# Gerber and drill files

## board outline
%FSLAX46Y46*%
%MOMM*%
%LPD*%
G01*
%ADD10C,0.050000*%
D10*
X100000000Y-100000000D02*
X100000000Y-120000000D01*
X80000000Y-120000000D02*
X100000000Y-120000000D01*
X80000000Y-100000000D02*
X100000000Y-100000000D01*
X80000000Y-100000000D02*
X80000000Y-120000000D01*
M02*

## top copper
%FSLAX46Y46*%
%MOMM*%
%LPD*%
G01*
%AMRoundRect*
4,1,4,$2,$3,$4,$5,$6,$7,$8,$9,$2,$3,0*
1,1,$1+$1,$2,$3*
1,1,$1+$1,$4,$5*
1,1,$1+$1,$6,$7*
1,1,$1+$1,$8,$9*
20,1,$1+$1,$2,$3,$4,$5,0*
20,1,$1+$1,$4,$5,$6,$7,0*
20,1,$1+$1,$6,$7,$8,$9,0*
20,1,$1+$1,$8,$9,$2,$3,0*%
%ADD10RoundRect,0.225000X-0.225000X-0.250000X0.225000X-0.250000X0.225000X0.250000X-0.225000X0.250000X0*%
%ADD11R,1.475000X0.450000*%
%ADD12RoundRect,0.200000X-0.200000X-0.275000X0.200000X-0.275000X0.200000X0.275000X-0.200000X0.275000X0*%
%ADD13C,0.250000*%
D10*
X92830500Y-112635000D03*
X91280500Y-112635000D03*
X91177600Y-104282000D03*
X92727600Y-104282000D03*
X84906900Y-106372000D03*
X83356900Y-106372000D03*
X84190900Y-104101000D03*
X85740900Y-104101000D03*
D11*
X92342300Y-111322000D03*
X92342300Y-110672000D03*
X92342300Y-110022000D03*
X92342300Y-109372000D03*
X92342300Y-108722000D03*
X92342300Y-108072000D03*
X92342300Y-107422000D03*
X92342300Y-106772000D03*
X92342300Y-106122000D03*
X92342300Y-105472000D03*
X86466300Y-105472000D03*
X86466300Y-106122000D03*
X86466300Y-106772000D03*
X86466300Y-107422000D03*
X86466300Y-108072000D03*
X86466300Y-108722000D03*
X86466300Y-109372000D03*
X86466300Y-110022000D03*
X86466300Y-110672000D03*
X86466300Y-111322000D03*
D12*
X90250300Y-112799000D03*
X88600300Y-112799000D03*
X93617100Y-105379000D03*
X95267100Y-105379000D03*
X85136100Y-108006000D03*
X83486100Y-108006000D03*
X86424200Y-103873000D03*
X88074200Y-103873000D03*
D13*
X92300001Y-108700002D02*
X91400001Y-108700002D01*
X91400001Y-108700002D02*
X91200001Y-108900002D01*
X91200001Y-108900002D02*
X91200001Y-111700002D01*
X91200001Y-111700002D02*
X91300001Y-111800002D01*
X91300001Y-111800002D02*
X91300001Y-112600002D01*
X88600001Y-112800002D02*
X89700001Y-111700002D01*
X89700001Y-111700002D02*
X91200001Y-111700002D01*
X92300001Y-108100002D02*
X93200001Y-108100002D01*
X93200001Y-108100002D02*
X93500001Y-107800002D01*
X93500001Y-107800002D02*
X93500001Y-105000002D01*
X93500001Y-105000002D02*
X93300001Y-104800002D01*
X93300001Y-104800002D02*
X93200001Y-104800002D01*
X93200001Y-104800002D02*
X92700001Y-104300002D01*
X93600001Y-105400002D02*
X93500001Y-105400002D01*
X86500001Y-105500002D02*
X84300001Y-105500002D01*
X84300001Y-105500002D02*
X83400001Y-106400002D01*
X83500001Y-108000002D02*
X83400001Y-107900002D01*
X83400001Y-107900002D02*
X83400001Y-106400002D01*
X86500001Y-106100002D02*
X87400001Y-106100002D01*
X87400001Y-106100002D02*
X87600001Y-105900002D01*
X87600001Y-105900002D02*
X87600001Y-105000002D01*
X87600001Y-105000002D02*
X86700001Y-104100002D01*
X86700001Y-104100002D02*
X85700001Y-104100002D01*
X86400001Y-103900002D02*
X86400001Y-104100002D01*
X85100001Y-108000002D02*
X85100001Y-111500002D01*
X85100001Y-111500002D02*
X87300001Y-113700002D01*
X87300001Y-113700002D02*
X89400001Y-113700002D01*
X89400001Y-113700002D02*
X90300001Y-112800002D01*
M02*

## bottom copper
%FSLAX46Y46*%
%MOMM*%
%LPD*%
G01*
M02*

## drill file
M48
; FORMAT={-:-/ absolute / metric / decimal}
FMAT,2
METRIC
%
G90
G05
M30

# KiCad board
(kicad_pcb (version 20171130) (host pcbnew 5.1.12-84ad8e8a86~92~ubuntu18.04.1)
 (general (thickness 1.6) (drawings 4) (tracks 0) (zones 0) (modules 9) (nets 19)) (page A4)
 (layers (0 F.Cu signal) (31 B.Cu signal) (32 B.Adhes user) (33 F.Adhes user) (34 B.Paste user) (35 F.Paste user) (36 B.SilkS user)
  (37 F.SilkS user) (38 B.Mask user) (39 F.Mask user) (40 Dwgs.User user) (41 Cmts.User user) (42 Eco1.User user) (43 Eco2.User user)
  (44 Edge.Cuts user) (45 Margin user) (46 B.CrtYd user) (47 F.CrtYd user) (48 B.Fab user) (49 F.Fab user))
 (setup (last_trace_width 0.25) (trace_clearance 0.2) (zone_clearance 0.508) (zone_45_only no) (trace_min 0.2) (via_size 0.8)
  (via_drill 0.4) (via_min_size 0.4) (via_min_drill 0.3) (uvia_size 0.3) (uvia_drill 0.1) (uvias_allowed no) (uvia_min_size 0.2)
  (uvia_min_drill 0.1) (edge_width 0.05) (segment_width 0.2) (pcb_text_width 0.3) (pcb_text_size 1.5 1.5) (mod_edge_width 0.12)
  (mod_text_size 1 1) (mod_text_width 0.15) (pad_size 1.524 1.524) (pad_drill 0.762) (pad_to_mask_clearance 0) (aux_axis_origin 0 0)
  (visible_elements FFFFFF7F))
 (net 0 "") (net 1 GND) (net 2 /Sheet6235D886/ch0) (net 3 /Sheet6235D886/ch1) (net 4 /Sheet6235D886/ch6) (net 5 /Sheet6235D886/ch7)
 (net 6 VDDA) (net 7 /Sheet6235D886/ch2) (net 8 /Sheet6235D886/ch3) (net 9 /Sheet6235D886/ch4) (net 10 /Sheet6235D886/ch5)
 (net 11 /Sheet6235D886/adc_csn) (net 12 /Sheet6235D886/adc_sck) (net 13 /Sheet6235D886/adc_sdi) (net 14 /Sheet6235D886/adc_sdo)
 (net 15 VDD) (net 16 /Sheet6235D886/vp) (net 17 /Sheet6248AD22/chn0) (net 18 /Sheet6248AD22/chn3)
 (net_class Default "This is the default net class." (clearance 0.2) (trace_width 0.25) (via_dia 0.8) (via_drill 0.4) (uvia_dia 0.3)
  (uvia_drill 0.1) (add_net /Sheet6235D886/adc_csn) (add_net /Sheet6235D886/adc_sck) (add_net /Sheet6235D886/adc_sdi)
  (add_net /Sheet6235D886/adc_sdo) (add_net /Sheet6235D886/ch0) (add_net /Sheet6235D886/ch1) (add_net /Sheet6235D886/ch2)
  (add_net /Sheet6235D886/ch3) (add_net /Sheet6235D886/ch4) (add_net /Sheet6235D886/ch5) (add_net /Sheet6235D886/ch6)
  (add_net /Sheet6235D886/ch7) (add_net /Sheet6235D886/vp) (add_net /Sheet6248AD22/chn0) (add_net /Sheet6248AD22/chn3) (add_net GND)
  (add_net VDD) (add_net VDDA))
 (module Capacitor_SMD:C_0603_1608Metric (layer F.Cu) (at 92.055500 112.635000)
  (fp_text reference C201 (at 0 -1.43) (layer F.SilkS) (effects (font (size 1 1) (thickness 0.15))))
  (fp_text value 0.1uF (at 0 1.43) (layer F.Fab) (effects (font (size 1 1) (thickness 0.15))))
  (pad 2 smd roundrect (at 0.775 0) (size 0.9 0.95) (layers F.Cu F.Mask F.Paste) (roundrect_rratio 0.25) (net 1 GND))
  (pad 1 smd roundrect (at -0.775 0) (size 0.9 0.95) (layers F.Cu F.Mask F.Paste) (roundrect_rratio 0.25) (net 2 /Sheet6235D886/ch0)))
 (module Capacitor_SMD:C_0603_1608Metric (layer F.Cu) (at 91.952600 104.282000)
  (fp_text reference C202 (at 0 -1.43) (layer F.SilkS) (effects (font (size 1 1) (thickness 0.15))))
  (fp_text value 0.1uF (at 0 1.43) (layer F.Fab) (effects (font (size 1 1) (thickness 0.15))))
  (pad 1 smd roundrect (at -0.775 0) (size 0.9 0.95) (layers F.Cu F.Mask F.Paste) (roundrect_rratio 0.25) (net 1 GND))
  (pad 2 smd roundrect (at 0.775 0) (size 0.9 0.95) (layers F.Cu F.Mask F.Paste) (roundrect_rratio 0.25) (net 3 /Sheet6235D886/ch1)))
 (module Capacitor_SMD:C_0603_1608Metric (layer F.Cu) (at 84.131900 106.372000)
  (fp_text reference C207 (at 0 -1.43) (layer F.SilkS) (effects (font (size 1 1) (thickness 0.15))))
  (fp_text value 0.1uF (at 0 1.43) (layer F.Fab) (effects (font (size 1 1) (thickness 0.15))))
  (pad 2 smd roundrect (at 0.775 0) (size 0.9 0.95) (layers F.Cu F.Mask F.Paste) (roundrect_rratio 0.25) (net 1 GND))
  (pad 1 smd roundrect (at -0.775 0) (size 0.9 0.95) (layers F.Cu F.Mask F.Paste) (roundrect_rratio 0.25) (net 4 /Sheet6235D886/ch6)))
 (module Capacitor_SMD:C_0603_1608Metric (layer F.Cu) (at 84.965900 104.101000)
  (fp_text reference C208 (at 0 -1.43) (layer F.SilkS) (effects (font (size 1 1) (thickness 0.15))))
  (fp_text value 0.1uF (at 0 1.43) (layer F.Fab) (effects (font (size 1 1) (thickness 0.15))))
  (pad 1 smd roundrect (at -0.775 0) (size 0.9 0.95) (layers F.Cu F.Mask F.Paste) (roundrect_rratio 0.25) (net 1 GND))
  (pad 2 smd roundrect (at 0.775 0) (size 0.9 0.95) (layers F.Cu F.Mask F.Paste) (roundrect_rratio 0.25) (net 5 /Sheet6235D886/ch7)))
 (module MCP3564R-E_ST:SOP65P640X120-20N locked (layer F.Cu) (at 89.404300 108.397000 180.000000)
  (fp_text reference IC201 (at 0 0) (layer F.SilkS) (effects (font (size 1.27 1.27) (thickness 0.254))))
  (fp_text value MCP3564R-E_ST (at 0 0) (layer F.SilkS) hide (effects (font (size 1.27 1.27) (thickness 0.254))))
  (pad 1 smd rect (at -2.938 -2.925 270.000000) (size 0.45 1.475) (layers F.Cu F.Mask F.Paste) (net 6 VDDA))
  (pad 2 smd rect (at -2.938 -2.275 270.000000) (size 0.45 1.475) (layers F.Cu F.Mask F.Paste) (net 1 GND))
  (pad 3 smd rect (at -2.938 -1.625 270.000000) (size 0.45 1.475) (layers F.Cu F.Mask F.Paste) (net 1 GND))
  (pad 4 smd rect (at -2.938 -0.975 270.000000) (size 0.45 1.475) (layers F.Cu F.Mask F.Paste))
  (pad 5 smd rect (at -2.938 -0.325 270.000000) (size 0.45 1.475) (layers F.Cu F.Mask F.Paste) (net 2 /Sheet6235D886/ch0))
  (pad 6 smd rect (at -2.938 0.325 270.000000) (size 0.45 1.475) (layers F.Cu F.Mask F.Paste) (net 3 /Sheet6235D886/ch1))
  (pad 7 smd rect (at -2.938 0.975 270.000000) (size 0.45 1.475) (layers F.Cu F.Mask F.Paste) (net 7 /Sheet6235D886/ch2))
  (pad 8 smd rect (at -2.938 1.625 270.000000) (size 0.45 1.475) (layers F.Cu F.Mask F.Paste) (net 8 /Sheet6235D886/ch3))
  (pad 9 smd rect (at -2.938 2.275 270.000000) (size 0.45 1.475) (layers F.Cu F.Mask F.Paste) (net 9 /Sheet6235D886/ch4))
  (pad 10 smd rect (at -2.938 2.925 270.000000) (size 0.45 1.475) (layers F.Cu F.Mask F.Paste) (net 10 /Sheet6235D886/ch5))
  (pad 11 smd rect (at 2.938 2.925 270.000000) (size 0.45 1.475) (layers F.Cu F.Mask F.Paste) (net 4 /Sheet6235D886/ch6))
  (pad 12 smd rect (at 2.938 2.275 270.000000) (size 0.45 1.475) (layers F.Cu F.Mask F.Paste) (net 5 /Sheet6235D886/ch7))
  (pad 13 smd rect (at 2.938 1.625 270.000000) (size 0.45 1.475) (layers F.Cu F.Mask F.Paste) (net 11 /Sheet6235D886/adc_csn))
  (pad 14 smd rect (at 2.938 0.975 270.000000) (size 0.45 1.475) (layers F.Cu F.Mask F.Paste) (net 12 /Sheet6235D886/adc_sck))
  (pad 15 smd rect (at 2.938 0.325 270.000000) (size 0.45 1.475) (layers F.Cu F.Mask F.Paste) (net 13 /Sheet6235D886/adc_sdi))
  (pad 16 smd rect (at 2.938 -0.325 270.000000) (size 0.45 1.475) (layers F.Cu F.Mask F.Paste) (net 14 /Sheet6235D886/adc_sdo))
  (pad 17 smd rect (at 2.938 -0.975 270.000000) (size 0.45 1.475) (layers F.Cu F.Mask F.Paste))
  (pad 18 smd rect (at 2.938 -1.625 270.000000) (size 0.45 1.475) (layers F.Cu F.Mask F.Paste))
  (pad 19 smd rect (at 2.938 -2.275 270.000000) (size 0.45 1.475) (layers F.Cu F.Mask F.Paste) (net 1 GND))
  (pad 20 smd rect (at 2.938 -2.925 270.000000) (size 0.45 1.475) (layers F.Cu F.Mask F.Paste) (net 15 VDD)))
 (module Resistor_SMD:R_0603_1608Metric (layer F.Cu) (at 89.425300 112.799000)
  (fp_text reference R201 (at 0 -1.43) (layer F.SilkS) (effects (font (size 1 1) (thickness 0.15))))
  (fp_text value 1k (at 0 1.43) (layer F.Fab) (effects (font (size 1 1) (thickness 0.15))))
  (pad 2 smd roundrect (at 0.825 0) (size 0.8 0.95) (layers F.Cu F.Mask F.Paste) (roundrect_rratio 0.25) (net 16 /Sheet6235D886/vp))
  (pad 1 smd roundrect (at -0.825 0) (size 0.8 0.95) (layers F.Cu F.Mask F.Paste) (roundrect_rratio 0.25) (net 2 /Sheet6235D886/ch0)))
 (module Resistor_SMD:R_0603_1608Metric (layer F.Cu) (at 94.442100 105.379000)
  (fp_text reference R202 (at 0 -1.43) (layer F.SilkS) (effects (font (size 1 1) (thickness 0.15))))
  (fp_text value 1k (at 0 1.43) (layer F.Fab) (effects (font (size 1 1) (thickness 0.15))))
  (pad 1 smd roundrect (at -0.825 0) (size 0.8 0.95) (layers F.Cu F.Mask F.Paste) (roundrect_rratio 0.25) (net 3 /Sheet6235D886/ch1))
  (pad 2 smd roundrect (at 0.825 0) (size 0.8 0.95) (layers F.Cu F.Mask F.Paste) (roundrect_rratio 0.25) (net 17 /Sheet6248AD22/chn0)))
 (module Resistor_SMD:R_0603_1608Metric (layer F.Cu) (at 84.311100 108.006000)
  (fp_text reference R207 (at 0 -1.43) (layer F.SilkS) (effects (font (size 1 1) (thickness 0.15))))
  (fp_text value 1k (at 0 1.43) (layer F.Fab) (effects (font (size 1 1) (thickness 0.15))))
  (pad 2 smd roundrect (at 0.825 0) (size 0.8 0.95) (layers F.Cu F.Mask F.Paste) (roundrect_rratio 0.25) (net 16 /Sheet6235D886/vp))
  (pad 1 smd roundrect (at -0.825 0) (size 0.8 0.95) (layers F.Cu F.Mask F.Paste) (roundrect_rratio 0.25) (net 4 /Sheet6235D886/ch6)))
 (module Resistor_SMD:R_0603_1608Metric (layer F.Cu) (at 87.249200 103.873000)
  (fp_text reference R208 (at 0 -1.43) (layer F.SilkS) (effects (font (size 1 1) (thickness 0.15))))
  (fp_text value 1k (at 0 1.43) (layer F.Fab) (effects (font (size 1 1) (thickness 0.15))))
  (pad 1 smd roundrect (at -0.825 0) (size 0.8 0.95) (layers F.Cu F.Mask F.Paste) (roundrect_rratio 0.25) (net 5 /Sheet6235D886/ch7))
  (pad 2 smd roundrect (at 0.825 0) (size 0.8 0.95) (layers F.Cu F.Mask F.Paste) (roundrect_rratio 0.25) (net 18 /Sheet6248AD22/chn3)))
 (gr_line (start 100 100) (end 100 120) (layer Edge.Cuts) (width 0.05))
 (gr_line (start 80 120) (end 100 120) (layer Edge.Cuts) (width 0.05))
 (gr_line (start 80 100) (end 100 100) (layer Edge.Cuts) (width 0.05))
 (gr_line (start 80 100) (end 80 120) (layer Edge.Cuts) (width 0.05))
 (segment (start 92.300001 108.700002) (end 91.400001 108.700002) (width 0.250000) (layer F.Cu) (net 2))
 (segment (start 91.400001 108.700002) (end 91.200001 108.900002) (width 0.250000) (layer F.Cu) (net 2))
 (segment (start 91.200001 108.900002) (end 91.200001 111.700002) (width 0.250000) (layer F.Cu) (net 2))
 (segment (start 91.200001 111.700002) (end 91.300001 111.800002) (width 0.250000) (layer F.Cu) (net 2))
 (segment (start 91.300001 111.800002) (end 91.300001 112.600002) (width 0.250000) (layer F.Cu) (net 2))
 (segment (start 88.600001 112.800002) (end 89.700001 111.700002) (width 0.250000) (layer F.Cu) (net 2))
 (segment (start 89.700001 111.700002) (end 91.200001 111.700002) (width 0.250000) (layer F.Cu) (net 2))
 (segment (start 92.300001 108.100002) (end 93.200001 108.100002) (width 0.250000) (layer F.Cu) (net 3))
 (segment (start 93.200001 108.100002) (end 93.500001 107.800002) (width 0.250000) (layer F.Cu) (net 3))
 (segment (start 93.500001 107.800002) (end 93.500001 105.000002) (width 0.250000) (layer F.Cu) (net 3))
 (segment (start 93.500001 105.000002) (end 93.300001 104.800002) (width 0.250000) (layer F.Cu) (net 3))
 (segment (start 93.300001 104.800002) (end 93.200001 104.800002) (width 0.250000) (layer F.Cu) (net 3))
 (segment (start 93.200001 104.800002) (end 92.700001 104.300002) (width 0.250000) (layer F.Cu) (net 3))
 (segment (start 93.600001 105.400002) (end 93.500001 105.400002) (width 0.250000) (layer F.Cu) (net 3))
 (segment (start 86.500001 105.500002) (end 84.300001 105.500002) (width 0.250000) (layer F.Cu) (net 4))
 (segment (start 84.300001 105.500002) (end 83.400001 106.400002) (width 0.250000) (layer F.Cu) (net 4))
 (segment (start 83.500001 108.000002) (end 83.400001 107.900002) (width 0.250000) (layer F.Cu) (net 4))
 (segment (start 83.400001 107.900002) (end 83.400001 106.400002) (width 0.250000) (layer F.Cu) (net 4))
 (segment (start 86.500001 106.100002) (end 87.400001 106.100002) (width 0.250000) (layer F.Cu) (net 5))
 (segment (start 87.400001 106.100002) (end 87.600001 105.900002) (width 0.250000) (layer F.Cu) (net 5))
 (segment (start 87.600001 105.900002) (end 87.600001 105.000002) (width 0.250000) (layer F.Cu) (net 5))
 (segment (start 87.600001 105.000002) (end 86.700001 104.100002) (width 0.250000) (layer F.Cu) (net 5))
 (segment (start 86.700001 104.100002) (end 85.700001 104.100002) (width 0.250000) (layer F.Cu) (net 5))
 (segment (start 86.400001 103.900002) (end 86.400001 104.100002) (width 0.250000) (layer F.Cu) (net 5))
 (segment (start 85.100001 108.000002) (end 85.100001 111.500002) (width 0.250000) (layer F.Cu) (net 16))
 (segment (start 85.100001 111.500002) (end 87.300001 113.700002) (width 0.250000) (layer F.Cu) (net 16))
 (segment (start 87.300001 113.700002) (end 89.400001 113.700002) (width 0.250000) (layer F.Cu) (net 16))
 (segment (start 89.400001 113.700002) (end 90.300001 112.800002) (width 0.250000) (layer F.Cu) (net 16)))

